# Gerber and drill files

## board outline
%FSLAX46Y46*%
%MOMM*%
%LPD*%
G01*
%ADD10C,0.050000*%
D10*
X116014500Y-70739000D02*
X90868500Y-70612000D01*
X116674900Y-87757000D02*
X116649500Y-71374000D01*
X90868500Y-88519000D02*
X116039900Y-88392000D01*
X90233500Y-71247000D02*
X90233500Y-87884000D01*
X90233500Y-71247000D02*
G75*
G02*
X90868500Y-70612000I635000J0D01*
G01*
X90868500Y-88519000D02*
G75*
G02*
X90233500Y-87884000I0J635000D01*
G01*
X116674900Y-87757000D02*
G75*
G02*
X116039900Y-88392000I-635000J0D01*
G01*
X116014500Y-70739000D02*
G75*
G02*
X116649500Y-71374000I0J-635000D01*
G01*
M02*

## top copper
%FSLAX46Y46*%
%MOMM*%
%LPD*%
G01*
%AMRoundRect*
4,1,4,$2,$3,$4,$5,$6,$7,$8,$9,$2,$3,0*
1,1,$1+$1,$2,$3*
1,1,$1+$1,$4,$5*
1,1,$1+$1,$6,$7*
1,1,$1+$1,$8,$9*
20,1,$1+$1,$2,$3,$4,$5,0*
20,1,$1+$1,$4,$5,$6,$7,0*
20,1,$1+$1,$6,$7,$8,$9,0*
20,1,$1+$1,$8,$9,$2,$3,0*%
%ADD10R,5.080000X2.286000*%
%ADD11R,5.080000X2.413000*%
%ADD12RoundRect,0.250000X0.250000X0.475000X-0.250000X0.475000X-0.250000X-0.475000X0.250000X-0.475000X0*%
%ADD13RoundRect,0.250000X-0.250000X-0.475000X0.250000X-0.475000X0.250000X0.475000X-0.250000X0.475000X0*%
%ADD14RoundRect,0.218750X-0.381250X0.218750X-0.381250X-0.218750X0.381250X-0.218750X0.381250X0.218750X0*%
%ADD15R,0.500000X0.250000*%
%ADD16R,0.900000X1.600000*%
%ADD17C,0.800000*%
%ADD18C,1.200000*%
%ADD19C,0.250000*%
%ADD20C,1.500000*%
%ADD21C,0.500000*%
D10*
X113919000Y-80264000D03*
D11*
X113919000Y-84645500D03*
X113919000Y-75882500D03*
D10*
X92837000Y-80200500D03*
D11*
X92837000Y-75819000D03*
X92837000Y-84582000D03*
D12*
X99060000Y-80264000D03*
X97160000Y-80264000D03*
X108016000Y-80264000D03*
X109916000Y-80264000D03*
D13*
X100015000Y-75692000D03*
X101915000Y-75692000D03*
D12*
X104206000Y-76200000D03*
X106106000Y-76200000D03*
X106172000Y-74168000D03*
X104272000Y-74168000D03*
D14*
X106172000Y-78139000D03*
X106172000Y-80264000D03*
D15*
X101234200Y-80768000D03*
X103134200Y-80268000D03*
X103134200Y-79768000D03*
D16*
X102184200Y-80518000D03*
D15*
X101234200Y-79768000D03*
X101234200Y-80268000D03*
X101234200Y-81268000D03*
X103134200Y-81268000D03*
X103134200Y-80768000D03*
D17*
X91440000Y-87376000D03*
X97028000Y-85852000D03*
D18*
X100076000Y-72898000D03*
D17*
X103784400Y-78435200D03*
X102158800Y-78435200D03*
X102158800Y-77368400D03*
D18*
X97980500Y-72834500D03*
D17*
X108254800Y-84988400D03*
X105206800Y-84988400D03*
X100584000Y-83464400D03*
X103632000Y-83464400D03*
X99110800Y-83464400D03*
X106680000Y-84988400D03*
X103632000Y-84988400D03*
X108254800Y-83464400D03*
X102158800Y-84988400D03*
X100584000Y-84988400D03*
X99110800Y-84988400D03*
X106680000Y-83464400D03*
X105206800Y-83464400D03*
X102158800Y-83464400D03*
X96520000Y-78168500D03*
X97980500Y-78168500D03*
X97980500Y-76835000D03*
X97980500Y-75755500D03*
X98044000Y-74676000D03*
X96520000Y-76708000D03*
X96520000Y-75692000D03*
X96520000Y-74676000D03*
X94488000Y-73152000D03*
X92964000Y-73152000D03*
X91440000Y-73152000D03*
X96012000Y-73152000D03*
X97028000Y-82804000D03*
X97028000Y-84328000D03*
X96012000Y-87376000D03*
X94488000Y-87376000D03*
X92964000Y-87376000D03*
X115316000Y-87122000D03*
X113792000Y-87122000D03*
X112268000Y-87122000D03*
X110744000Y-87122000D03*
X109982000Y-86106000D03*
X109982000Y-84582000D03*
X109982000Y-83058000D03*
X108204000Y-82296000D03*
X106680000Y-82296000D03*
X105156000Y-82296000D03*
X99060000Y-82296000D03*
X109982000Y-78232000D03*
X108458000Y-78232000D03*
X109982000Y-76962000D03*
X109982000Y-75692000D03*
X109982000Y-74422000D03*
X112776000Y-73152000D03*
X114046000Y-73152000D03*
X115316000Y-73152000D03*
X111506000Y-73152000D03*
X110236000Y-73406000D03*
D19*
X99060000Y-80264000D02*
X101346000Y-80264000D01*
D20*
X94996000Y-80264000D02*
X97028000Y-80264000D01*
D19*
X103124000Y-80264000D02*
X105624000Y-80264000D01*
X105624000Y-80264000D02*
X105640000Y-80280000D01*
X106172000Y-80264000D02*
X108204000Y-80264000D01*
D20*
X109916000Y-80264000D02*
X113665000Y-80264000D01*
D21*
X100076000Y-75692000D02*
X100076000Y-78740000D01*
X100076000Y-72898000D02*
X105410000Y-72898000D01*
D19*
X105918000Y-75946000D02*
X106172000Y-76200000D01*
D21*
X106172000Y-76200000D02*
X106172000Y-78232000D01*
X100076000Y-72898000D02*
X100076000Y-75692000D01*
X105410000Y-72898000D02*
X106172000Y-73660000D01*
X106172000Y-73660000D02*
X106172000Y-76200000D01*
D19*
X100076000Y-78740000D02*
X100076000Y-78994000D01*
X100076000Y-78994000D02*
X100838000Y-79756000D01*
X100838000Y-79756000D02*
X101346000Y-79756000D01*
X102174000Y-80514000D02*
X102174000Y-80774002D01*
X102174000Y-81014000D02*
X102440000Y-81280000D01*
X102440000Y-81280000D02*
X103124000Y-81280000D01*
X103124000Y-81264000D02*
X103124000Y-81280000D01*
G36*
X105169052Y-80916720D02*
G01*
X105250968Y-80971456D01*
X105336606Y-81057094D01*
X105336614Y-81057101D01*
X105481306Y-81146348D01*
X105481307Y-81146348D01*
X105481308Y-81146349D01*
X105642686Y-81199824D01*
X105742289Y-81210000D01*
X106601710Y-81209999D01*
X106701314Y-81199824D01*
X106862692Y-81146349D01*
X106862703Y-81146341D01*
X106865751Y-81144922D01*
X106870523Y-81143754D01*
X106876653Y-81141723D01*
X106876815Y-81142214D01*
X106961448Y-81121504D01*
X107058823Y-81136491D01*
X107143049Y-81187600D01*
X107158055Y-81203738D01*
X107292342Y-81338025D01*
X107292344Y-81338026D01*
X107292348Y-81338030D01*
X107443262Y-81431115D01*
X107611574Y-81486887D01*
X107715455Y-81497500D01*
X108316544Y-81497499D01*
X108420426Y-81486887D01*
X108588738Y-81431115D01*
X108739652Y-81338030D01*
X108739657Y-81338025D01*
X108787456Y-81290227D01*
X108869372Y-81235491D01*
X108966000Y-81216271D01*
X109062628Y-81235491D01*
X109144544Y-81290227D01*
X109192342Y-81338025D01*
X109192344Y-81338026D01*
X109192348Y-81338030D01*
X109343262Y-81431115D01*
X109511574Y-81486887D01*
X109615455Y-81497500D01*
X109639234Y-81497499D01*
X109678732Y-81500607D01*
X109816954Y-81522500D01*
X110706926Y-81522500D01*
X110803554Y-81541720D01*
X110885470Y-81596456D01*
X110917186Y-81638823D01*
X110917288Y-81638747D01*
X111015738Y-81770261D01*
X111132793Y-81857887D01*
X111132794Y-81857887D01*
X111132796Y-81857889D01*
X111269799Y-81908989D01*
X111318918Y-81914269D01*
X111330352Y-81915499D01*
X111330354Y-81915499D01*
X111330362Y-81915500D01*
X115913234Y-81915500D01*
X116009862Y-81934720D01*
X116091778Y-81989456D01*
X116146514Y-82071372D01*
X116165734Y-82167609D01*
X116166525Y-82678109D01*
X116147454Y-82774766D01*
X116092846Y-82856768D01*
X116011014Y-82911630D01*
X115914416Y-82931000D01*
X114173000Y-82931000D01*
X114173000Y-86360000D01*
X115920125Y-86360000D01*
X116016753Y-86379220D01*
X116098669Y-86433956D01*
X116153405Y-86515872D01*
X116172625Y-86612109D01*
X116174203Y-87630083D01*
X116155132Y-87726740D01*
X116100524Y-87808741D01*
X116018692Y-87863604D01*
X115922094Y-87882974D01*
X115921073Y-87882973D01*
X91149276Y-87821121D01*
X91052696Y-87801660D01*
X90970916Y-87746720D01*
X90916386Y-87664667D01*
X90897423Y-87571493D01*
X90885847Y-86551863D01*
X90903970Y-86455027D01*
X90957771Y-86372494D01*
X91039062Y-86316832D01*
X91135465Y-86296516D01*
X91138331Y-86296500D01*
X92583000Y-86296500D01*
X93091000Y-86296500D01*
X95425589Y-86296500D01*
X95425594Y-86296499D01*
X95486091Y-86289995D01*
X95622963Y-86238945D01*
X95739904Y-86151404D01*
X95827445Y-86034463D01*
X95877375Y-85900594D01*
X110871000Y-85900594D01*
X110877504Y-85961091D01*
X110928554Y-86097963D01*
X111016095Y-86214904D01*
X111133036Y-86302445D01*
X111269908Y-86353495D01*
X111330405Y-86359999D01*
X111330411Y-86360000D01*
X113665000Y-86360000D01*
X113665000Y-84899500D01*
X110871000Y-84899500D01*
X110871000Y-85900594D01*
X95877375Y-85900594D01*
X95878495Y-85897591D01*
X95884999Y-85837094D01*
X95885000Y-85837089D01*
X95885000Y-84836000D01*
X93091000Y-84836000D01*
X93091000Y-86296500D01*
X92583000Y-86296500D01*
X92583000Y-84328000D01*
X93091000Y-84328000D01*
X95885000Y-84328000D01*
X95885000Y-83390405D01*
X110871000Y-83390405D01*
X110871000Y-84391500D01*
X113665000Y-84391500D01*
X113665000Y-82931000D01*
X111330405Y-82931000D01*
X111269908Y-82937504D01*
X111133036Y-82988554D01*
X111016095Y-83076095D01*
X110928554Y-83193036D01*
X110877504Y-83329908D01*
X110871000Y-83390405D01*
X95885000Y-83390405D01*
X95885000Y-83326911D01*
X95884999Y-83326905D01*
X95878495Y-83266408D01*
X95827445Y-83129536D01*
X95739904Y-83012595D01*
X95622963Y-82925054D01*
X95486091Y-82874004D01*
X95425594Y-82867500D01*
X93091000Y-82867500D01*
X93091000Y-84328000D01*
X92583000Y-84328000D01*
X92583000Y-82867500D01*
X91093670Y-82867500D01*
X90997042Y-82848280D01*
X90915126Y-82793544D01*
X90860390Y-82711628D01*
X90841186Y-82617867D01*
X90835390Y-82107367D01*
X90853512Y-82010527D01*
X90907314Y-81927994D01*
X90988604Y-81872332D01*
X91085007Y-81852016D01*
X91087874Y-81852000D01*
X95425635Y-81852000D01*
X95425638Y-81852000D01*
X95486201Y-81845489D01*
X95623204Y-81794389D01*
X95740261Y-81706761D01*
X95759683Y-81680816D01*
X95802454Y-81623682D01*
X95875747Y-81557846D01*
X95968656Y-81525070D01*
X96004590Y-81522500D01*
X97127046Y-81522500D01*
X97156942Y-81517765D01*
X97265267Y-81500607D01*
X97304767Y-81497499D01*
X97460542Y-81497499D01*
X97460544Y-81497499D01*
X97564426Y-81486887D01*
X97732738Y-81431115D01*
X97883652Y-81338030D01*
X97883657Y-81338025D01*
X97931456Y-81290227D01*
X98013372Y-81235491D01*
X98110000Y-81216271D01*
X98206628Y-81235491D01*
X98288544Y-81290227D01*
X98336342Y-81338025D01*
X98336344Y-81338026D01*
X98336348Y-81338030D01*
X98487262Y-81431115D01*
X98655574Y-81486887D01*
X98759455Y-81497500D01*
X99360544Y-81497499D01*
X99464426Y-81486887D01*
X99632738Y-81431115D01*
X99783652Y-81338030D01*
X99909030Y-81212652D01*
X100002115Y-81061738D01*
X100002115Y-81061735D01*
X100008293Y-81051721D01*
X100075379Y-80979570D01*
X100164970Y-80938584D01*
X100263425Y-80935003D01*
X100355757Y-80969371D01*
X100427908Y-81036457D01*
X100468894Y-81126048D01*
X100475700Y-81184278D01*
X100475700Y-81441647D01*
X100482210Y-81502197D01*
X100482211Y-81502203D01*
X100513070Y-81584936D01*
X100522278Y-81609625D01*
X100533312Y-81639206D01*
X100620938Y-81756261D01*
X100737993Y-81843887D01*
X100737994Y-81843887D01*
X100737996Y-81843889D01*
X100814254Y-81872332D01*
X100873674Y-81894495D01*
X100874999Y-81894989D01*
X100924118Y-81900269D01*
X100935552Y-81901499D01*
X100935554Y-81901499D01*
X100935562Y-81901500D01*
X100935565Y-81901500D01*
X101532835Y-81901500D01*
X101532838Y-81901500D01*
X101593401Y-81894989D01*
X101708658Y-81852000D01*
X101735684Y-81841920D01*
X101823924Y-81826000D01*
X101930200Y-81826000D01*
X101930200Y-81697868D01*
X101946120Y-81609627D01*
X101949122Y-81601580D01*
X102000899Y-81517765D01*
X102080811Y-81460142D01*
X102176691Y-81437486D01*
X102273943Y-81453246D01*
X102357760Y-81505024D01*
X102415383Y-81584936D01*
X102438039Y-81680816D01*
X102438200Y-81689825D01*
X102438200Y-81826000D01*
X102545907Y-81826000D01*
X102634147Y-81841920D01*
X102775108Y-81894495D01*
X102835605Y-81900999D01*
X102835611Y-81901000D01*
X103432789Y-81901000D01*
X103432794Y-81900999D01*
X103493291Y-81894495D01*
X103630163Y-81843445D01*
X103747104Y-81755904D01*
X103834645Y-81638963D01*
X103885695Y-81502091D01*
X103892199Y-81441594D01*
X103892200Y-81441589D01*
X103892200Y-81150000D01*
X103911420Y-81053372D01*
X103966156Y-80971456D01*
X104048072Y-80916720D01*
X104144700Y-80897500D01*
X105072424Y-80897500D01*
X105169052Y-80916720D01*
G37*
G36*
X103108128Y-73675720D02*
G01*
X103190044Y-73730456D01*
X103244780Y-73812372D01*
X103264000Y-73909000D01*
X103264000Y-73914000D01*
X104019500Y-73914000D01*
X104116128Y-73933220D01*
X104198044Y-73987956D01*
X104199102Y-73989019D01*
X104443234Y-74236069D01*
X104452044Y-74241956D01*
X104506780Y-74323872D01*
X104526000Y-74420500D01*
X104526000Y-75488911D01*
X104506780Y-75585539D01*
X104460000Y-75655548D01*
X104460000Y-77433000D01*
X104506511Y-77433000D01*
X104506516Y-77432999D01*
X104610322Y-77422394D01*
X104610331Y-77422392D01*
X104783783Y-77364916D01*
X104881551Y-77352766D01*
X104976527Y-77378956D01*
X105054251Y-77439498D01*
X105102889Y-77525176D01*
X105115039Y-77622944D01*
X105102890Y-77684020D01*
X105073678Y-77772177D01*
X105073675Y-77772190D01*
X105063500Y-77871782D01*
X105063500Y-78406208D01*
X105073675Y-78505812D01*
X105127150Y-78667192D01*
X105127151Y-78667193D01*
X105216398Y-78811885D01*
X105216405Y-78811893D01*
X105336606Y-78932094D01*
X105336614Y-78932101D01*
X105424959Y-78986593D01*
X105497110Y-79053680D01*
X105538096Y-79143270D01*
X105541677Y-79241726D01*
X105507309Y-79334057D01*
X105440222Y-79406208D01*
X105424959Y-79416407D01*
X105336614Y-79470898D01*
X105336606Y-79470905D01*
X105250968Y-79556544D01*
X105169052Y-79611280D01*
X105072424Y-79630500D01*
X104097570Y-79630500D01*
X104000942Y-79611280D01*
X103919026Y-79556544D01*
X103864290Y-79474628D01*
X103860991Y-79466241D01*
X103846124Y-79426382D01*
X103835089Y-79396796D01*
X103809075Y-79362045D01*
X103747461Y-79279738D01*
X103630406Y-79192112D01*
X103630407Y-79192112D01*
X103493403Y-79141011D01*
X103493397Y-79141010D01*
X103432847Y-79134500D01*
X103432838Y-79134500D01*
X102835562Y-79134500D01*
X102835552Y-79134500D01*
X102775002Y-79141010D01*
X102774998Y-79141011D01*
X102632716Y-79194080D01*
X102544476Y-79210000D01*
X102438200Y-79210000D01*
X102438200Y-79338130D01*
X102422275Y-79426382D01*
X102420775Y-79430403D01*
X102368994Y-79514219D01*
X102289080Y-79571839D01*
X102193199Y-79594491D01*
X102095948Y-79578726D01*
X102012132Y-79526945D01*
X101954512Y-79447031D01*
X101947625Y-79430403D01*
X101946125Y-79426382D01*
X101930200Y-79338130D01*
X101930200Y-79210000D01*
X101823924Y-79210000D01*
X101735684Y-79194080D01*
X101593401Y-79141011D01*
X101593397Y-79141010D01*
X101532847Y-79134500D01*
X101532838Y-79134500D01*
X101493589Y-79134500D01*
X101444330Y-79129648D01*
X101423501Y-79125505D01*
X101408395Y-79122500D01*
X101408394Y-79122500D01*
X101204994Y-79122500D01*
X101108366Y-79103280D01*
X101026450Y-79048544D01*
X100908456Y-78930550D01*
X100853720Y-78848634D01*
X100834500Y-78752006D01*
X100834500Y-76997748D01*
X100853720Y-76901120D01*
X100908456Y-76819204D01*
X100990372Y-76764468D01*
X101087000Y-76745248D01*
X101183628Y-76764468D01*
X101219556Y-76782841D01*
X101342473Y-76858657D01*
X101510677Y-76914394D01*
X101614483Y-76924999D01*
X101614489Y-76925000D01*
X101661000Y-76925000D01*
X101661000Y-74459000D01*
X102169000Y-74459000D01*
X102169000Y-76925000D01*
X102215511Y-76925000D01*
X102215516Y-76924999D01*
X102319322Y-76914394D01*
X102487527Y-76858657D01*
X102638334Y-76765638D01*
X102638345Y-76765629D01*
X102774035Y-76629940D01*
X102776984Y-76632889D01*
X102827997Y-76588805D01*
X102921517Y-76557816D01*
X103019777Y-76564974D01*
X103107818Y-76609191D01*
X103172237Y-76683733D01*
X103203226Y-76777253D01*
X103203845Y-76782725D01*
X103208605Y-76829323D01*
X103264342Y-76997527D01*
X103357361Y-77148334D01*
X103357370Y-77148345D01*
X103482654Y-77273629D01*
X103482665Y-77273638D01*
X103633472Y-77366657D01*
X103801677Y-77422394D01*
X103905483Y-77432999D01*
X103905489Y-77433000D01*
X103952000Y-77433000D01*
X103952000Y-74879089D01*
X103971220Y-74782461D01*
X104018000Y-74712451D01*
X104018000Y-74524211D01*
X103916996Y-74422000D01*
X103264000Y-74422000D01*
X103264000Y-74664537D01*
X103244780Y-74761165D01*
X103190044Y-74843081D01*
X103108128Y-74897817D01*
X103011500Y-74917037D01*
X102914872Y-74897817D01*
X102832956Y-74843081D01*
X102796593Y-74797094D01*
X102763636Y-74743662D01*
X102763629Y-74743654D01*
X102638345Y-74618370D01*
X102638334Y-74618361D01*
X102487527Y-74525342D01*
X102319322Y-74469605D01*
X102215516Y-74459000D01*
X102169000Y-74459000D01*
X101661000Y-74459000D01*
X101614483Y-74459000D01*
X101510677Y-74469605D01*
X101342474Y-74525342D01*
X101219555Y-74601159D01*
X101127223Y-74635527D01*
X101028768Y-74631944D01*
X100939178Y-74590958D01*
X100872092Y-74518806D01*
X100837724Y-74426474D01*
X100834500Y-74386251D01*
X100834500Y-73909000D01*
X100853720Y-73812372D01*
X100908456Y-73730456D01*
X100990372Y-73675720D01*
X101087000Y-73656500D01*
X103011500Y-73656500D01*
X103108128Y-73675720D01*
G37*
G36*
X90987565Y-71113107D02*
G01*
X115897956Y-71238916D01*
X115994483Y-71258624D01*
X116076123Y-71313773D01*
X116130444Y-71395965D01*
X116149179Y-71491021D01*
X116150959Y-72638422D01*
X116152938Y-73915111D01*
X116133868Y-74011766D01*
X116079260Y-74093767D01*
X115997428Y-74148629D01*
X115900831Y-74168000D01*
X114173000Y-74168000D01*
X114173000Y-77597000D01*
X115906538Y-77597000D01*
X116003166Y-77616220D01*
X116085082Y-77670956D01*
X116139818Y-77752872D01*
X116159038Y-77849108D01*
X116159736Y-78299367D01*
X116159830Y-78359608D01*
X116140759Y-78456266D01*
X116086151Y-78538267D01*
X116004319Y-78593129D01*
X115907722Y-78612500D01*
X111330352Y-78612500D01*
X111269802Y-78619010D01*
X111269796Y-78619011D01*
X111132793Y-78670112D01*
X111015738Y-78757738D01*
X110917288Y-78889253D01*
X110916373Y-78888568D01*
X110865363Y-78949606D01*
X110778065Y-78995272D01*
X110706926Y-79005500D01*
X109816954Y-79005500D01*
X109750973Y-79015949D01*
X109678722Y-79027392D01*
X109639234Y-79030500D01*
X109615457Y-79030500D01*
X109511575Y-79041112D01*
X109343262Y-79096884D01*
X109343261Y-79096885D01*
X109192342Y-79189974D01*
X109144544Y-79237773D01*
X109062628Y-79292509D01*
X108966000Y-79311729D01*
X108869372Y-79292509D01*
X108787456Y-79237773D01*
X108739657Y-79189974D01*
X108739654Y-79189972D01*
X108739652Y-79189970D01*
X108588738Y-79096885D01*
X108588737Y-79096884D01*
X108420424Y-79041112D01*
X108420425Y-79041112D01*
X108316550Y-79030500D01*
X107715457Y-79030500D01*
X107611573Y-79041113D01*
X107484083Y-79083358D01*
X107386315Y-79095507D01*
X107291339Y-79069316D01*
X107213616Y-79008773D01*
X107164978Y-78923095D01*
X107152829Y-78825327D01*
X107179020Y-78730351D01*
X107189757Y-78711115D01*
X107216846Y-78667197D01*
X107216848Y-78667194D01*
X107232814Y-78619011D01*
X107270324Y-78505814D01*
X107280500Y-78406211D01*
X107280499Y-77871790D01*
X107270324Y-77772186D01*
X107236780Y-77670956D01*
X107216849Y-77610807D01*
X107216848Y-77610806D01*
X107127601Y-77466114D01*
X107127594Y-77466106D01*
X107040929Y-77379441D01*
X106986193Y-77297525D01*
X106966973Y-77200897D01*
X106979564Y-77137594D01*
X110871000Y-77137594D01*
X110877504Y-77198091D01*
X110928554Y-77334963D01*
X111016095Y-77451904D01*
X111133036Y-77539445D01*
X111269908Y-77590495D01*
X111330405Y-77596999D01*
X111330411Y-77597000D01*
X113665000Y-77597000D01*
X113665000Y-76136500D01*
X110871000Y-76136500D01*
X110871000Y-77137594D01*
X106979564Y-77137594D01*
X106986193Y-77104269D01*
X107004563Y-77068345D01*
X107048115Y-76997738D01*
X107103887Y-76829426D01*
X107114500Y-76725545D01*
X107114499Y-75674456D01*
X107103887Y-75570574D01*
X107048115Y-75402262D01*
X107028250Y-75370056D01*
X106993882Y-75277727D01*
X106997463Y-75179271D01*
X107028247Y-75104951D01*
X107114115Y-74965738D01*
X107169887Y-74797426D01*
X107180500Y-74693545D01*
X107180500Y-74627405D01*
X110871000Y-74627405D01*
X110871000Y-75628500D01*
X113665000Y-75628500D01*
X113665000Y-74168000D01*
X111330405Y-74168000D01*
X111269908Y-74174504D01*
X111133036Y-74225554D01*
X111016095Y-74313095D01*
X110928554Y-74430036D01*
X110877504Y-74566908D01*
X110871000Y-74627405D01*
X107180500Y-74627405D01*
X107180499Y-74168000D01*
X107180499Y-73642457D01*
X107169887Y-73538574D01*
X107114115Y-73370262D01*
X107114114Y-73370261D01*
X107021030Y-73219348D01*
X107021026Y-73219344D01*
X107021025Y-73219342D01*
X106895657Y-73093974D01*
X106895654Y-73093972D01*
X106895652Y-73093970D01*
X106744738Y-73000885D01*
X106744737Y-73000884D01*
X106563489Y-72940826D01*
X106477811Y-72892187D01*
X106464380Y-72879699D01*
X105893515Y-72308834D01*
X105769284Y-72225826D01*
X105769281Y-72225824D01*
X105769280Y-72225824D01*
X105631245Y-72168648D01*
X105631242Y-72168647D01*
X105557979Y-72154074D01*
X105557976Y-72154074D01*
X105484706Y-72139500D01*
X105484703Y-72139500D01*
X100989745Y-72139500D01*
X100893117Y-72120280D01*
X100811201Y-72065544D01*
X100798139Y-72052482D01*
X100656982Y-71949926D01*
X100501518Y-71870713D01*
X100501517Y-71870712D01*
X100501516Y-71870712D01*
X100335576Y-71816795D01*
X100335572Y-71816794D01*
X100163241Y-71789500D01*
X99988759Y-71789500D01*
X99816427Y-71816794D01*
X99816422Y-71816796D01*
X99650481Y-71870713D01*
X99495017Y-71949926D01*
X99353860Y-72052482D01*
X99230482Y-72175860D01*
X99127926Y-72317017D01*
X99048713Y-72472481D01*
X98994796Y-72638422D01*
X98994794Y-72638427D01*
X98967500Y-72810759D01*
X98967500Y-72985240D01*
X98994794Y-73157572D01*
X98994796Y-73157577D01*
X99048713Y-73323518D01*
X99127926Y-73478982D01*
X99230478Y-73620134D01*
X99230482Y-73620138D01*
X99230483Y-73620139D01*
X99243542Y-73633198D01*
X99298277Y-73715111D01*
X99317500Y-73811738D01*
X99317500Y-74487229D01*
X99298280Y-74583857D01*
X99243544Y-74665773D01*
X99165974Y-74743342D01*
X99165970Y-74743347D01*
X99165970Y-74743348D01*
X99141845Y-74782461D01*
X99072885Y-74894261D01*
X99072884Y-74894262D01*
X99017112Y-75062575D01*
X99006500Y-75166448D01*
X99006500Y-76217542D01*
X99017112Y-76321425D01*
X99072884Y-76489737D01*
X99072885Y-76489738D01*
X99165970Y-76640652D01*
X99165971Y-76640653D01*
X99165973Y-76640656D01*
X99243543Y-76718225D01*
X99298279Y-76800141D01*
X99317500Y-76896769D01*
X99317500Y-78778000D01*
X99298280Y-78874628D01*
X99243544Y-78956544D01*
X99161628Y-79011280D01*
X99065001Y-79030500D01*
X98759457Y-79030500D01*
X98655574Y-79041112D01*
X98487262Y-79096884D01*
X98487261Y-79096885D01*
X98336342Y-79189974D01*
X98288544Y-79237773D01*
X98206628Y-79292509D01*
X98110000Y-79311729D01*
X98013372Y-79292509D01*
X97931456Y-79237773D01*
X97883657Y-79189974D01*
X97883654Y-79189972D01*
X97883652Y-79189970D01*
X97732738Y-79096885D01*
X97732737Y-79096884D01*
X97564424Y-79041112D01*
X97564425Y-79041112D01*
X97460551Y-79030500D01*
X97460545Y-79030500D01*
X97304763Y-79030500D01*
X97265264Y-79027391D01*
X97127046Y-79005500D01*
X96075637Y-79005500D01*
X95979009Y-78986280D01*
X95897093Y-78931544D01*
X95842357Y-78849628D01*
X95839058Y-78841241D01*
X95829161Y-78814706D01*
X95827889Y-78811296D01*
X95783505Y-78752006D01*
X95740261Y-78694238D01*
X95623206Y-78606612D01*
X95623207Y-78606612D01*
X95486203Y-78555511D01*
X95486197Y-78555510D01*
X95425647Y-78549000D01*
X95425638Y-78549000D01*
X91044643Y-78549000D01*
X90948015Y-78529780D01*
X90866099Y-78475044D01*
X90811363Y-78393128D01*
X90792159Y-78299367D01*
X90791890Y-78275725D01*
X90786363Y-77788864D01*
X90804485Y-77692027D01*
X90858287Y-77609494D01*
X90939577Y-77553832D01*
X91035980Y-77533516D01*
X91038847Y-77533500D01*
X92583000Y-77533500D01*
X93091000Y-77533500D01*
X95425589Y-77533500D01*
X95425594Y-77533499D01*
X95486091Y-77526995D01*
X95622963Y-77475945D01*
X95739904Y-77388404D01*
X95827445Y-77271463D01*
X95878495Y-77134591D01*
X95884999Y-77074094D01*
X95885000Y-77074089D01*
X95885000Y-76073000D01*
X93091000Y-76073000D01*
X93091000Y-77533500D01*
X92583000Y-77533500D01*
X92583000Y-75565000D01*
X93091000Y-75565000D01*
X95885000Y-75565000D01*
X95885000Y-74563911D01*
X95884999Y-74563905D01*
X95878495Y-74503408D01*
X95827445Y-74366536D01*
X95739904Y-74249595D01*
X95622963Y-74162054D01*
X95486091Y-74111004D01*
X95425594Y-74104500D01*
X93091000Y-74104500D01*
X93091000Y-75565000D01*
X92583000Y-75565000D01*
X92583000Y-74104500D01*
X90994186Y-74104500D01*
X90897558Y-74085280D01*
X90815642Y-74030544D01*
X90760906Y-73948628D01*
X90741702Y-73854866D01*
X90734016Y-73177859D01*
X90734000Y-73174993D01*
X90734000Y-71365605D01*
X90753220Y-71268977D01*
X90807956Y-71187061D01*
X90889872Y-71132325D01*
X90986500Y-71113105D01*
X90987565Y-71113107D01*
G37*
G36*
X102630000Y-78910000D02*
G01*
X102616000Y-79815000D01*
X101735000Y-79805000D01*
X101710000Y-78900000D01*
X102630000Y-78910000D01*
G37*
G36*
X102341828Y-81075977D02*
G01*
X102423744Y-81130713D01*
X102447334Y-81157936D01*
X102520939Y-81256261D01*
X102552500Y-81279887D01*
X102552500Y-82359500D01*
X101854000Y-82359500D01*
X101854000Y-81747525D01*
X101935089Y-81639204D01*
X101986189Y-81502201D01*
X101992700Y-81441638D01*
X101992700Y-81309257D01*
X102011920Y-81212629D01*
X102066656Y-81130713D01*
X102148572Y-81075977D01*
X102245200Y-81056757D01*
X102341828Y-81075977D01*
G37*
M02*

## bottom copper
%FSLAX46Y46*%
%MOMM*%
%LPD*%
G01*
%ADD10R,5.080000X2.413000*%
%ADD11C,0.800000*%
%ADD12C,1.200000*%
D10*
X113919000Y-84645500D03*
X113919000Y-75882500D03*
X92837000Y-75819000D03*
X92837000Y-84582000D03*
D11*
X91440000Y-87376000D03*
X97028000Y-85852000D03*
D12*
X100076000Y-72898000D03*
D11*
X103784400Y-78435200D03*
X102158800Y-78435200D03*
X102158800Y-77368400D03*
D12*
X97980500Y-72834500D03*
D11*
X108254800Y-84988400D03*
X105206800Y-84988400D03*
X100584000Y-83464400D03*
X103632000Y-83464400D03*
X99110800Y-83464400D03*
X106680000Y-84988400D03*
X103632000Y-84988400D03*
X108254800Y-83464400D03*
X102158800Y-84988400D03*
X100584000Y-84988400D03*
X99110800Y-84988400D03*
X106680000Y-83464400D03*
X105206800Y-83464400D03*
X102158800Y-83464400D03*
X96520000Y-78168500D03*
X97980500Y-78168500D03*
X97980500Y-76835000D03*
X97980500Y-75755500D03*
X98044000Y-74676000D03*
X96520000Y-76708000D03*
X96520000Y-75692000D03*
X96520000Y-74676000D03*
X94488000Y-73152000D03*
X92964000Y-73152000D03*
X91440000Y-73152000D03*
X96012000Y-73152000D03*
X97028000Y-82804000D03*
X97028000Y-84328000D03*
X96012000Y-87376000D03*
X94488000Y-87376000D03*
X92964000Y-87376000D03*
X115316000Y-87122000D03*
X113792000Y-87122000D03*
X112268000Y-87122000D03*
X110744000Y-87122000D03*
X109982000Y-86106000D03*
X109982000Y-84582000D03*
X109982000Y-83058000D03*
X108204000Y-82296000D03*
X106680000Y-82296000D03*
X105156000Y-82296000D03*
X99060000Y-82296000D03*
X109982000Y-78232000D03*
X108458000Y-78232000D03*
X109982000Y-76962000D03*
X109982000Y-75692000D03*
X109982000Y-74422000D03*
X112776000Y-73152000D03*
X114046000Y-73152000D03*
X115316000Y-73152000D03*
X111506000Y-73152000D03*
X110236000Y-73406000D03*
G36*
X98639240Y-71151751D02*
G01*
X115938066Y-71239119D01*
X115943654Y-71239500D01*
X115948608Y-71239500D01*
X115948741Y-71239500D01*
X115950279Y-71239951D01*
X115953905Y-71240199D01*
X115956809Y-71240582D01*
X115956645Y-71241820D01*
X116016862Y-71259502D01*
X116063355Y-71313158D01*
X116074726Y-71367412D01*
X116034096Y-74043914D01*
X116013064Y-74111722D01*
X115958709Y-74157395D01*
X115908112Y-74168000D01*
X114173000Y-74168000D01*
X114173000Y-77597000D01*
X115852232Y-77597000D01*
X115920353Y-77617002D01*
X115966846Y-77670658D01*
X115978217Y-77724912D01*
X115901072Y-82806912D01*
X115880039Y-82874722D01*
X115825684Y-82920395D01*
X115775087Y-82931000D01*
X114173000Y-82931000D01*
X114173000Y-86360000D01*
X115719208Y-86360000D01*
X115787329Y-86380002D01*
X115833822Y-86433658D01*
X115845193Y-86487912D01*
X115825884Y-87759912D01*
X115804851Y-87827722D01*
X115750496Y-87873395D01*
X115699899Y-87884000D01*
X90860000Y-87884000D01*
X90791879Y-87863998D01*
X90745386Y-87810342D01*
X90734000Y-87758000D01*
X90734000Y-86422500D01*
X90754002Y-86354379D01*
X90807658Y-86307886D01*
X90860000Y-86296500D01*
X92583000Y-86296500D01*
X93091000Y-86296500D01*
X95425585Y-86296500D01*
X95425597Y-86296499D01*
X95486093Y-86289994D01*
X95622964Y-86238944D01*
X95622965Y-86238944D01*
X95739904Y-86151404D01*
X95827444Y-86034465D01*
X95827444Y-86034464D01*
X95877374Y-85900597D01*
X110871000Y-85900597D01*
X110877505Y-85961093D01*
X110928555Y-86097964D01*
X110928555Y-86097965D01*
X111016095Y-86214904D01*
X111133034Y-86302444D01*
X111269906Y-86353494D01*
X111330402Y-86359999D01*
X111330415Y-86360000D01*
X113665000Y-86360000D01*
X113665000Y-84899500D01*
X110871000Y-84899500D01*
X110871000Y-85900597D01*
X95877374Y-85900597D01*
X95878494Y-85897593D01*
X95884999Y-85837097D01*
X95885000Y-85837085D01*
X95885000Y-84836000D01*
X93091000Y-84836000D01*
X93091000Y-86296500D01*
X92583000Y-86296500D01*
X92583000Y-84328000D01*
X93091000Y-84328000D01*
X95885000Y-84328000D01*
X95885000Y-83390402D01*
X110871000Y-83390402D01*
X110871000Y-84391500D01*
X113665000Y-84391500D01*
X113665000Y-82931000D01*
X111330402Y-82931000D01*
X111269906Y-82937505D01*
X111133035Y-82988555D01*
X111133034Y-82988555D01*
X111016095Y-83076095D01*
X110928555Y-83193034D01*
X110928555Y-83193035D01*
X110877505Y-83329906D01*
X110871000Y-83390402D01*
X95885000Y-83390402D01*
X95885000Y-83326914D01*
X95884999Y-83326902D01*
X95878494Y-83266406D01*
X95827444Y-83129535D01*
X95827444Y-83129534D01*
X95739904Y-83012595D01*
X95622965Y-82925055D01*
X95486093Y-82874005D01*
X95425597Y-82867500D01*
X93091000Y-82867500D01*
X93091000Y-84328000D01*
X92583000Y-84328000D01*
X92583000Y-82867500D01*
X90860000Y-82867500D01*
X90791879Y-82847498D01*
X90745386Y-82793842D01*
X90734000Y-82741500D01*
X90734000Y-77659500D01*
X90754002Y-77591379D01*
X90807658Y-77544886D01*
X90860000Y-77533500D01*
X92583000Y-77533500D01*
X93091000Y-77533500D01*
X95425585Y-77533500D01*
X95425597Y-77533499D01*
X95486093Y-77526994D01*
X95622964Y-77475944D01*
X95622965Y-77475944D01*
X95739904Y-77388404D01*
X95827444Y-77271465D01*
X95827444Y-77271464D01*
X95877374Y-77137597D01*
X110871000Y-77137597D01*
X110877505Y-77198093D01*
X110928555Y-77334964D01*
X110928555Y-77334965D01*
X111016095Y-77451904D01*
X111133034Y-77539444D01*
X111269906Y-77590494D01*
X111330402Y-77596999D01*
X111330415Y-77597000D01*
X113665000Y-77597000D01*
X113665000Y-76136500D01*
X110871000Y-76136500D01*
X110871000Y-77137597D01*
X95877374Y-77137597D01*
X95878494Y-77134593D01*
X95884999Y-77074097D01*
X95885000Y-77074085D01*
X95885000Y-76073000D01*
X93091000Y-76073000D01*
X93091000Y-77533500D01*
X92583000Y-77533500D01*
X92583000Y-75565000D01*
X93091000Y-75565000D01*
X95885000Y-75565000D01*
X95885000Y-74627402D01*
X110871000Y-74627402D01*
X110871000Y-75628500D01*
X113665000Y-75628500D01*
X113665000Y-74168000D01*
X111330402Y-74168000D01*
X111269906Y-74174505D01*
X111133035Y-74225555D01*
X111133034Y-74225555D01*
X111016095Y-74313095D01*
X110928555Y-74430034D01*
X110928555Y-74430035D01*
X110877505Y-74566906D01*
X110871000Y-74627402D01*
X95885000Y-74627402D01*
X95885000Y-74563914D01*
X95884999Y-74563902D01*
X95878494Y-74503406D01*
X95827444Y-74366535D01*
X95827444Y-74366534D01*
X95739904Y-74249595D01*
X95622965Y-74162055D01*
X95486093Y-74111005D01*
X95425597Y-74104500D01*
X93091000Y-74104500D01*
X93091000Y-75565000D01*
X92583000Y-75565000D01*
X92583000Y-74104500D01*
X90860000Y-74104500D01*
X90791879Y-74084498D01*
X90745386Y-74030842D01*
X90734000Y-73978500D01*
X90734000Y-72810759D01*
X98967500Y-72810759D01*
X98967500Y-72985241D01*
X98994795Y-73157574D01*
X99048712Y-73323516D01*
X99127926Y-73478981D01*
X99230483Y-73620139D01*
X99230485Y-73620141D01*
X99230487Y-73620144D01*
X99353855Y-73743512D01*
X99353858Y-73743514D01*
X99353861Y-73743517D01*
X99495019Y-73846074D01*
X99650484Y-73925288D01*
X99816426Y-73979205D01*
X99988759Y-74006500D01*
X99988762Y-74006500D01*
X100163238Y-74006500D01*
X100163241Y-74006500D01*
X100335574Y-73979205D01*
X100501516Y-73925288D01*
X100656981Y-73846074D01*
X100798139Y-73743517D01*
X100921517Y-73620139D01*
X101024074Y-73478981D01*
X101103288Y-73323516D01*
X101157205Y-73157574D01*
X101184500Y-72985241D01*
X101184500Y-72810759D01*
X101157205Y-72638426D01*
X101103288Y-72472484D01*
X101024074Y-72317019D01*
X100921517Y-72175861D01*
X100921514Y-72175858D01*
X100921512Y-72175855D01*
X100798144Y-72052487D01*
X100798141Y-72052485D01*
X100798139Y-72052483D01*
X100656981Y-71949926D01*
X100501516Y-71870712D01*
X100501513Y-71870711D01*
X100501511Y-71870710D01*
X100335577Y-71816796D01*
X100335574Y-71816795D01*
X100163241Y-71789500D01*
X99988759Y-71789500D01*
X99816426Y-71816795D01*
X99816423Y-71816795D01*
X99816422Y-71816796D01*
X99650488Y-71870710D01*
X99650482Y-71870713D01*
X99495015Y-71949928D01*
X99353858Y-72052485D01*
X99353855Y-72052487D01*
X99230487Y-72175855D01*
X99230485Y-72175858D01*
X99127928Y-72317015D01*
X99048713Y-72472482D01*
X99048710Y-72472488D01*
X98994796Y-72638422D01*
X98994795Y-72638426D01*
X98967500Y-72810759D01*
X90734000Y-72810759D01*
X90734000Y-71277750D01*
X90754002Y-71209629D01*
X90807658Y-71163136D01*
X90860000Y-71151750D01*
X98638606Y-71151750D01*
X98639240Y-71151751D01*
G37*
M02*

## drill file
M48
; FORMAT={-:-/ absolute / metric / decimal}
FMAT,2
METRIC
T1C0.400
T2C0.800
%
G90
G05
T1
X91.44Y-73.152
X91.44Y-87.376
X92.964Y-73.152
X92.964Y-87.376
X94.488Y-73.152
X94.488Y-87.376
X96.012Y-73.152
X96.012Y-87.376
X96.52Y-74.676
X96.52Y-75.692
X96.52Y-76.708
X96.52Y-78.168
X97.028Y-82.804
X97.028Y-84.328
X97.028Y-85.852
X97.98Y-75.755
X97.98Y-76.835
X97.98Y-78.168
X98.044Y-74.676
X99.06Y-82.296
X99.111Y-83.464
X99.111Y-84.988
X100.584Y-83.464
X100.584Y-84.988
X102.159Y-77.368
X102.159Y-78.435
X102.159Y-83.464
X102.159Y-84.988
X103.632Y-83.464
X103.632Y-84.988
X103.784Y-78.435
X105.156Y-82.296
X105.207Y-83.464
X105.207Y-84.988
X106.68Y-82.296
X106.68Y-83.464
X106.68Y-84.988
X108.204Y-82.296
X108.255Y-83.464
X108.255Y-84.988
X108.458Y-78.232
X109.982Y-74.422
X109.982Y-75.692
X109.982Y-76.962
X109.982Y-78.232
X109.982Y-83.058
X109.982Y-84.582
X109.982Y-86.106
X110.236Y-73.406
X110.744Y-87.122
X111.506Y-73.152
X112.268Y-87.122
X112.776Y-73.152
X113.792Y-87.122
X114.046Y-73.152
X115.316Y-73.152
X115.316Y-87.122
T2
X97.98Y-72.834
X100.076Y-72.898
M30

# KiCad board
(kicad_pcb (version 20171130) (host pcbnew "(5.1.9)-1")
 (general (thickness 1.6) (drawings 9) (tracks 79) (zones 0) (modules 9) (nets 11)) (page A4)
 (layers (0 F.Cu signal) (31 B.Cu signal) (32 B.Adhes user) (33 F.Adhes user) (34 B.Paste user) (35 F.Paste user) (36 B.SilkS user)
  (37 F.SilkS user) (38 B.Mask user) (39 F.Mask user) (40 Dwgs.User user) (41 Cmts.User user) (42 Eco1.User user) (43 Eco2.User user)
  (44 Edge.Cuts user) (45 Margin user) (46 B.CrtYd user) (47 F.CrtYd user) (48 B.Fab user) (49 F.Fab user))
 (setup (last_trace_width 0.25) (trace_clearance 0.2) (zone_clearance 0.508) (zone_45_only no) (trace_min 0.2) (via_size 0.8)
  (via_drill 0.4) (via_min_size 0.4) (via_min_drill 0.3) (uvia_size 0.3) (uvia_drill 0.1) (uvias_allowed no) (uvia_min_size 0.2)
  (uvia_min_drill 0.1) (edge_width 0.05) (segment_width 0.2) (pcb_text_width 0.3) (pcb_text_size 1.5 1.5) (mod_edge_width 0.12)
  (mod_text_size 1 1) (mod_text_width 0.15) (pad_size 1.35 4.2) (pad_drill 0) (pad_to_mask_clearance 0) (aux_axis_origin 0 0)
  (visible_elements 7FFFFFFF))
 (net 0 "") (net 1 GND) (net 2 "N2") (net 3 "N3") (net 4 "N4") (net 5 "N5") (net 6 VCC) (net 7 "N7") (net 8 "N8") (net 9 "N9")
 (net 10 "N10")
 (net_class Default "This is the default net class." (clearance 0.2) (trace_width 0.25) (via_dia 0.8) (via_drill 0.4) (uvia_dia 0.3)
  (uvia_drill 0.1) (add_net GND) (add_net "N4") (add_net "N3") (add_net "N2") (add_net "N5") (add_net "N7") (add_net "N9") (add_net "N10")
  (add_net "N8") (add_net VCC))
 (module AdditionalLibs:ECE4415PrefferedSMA (layer F.Cu) (at 113.919 80.264 270)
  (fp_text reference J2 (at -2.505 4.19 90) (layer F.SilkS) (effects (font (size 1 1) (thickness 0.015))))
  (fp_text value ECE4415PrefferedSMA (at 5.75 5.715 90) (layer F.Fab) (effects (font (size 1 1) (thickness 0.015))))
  (pad S4 smd rect (at 4.3815 0 270) (size 2.413 5.08) (layers B.Cu B.Paste B.Mask) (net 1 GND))
  (pad S3 smd rect (at -4.3815 0 270) (size 2.413 5.08) (layers B.Cu B.Paste B.Mask) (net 1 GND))
  (pad 1 smd rect (at 0 0 270) (size 2.286 5.08) (layers F.Cu F.Paste F.Mask) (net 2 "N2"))
  (pad S2 smd rect (at 4.3815 0 270) (size 2.413 5.08) (layers F.Cu F.Paste F.Mask) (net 1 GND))
  (pad S1 smd rect (at -4.3815 0 270) (size 2.413 5.08) (layers F.Cu F.Paste F.Mask) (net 1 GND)))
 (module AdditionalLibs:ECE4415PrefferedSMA (layer F.Cu) (at 92.837 80.2005 90)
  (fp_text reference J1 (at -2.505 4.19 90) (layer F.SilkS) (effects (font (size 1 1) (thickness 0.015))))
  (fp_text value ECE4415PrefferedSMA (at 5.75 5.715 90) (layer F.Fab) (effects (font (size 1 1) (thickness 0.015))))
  (pad S4 smd rect (at 4.3815 0 90) (size 2.413 5.08) (layers B.Cu B.Paste B.Mask) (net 1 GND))
  (pad S3 smd rect (at -4.3815 0 90) (size 2.413 5.08) (layers B.Cu B.Paste B.Mask) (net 1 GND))
  (pad 1 smd rect (at 0 0 90) (size 2.286 5.08) (layers F.Cu F.Paste F.Mask) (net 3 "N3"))
  (pad S2 smd rect (at 4.3815 0 90) (size 2.413 5.08) (layers F.Cu F.Paste F.Mask) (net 1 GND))
  (pad S1 smd rect (at -4.3815 0 90) (size 2.413 5.08) (layers F.Cu F.Paste F.Mask) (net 1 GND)))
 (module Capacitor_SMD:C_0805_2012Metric (layer F.Cu) (at 98.11 80.264 180)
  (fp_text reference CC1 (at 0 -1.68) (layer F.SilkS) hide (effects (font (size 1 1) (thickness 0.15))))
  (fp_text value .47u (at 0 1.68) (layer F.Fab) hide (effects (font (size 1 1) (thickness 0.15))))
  (pad 1 smd roundrect (at -0.95 0 180) (size 1 1.45) (layers F.Cu F.Paste F.Mask) (roundrect_rratio 0.25) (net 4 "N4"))
  (pad 2 smd roundrect (at 0.95 0 180) (size 1 1.45) (layers F.Cu F.Paste F.Mask) (roundrect_rratio 0.25) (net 3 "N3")))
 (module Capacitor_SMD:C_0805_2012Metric (layer F.Cu) (at 108.966 80.264 180)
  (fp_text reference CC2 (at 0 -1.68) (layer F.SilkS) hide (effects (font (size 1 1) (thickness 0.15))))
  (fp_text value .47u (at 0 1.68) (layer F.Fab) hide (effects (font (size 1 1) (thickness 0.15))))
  (pad 2 smd roundrect (at 0.95 0 180) (size 1 1.45) (layers F.Cu F.Paste F.Mask) (roundrect_rratio 0.25) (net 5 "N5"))
  (pad 1 smd roundrect (at -0.95 0 180) (size 1 1.45) (layers F.Cu F.Paste F.Mask) (roundrect_rratio 0.25) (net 2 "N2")))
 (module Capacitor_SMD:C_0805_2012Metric (layer F.Cu) (at 100.965 75.692)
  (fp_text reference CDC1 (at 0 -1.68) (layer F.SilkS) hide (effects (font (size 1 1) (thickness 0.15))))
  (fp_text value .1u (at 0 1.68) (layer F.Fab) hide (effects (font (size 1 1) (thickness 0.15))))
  (pad 1 smd roundrect (at -0.95 0) (size 1 1.45) (layers F.Cu F.Paste F.Mask) (roundrect_rratio 0.25) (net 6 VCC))
  (pad 2 smd roundrect (at 0.95 0) (size 1 1.45) (layers F.Cu F.Paste F.Mask) (roundrect_rratio 0.25) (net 1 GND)))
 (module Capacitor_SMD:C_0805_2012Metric (layer F.Cu) (at 105.156 76.2 180)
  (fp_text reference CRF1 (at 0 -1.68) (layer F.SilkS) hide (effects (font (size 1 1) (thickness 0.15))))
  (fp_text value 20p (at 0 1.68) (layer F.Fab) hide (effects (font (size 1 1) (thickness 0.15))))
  (pad 2 smd roundrect (at 0.95 0 180) (size 1 1.45) (layers F.Cu F.Paste F.Mask) (roundrect_rratio 0.25) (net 1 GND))
  (pad 1 smd roundrect (at -0.95 0 180) (size 1 1.45) (layers F.Cu F.Paste F.Mask) (roundrect_rratio 0.25) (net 6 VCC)))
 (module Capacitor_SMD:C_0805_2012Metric (layer F.Cu) (at 105.222 74.168 180)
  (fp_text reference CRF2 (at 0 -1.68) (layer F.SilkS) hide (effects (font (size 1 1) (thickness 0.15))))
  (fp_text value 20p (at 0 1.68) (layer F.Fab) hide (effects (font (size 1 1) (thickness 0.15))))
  (pad 1 smd roundrect (at -0.95 0 180) (size 1 1.45) (layers F.Cu F.Paste F.Mask) (roundrect_rratio 0.25) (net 6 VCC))
  (pad 2 smd roundrect (at 0.95 0 180) (size 1 1.45) (layers F.Cu F.Paste F.Mask) (roundrect_rratio 0.25) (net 1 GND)))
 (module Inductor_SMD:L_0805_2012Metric (layer F.Cu) (at 106.172 79.2015 270)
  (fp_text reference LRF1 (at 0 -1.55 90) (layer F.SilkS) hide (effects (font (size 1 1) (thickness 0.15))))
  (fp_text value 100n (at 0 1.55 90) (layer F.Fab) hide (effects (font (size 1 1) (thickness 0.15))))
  (pad 1 smd roundrect (at -1.0625 0 270) (size 0.875 1.2) (layers F.Cu F.Paste F.Mask) (roundrect_rratio 0.25) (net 6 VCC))
  (pad 2 smd roundrect (at 1.0625 0 270) (size 0.875 1.2) (layers F.Cu F.Paste F.Mask) (roundrect_rratio 0.25) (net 5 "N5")))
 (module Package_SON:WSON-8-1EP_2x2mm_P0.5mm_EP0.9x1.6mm (layer F.Cu) (at 102.1842 80.518)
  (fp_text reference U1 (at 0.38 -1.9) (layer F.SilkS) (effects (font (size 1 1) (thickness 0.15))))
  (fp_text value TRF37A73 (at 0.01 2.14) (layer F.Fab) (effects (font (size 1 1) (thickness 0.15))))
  (pad 3 smd rect (at -0.95 0.25) (size 0.5 0.25) (layers F.Cu F.Paste F.Mask) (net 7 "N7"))
  (pad 7 smd rect (at 0.95 -0.25) (size 0.5 0.25) (layers F.Cu F.Paste F.Mask) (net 5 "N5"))
  (pad 8 smd rect (at 0.95 -0.75) (size 0.5 0.25) (layers F.Cu F.Paste F.Mask) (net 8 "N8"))
  (pad 9 smd rect (at 0 0) (size 0.9 1.6) (layers F.Cu F.Mask) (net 1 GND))
  (pad 1 smd rect (at -0.95 -0.75) (size 0.5 0.25) (layers F.Cu F.Paste F.Mask) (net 6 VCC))
  (pad 2 smd rect (at -0.95 -0.25) (size 0.5 0.25) (layers F.Cu F.Paste F.Mask) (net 4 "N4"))
  (pad 4 smd rect (at -0.95 0.75) (size 0.5 0.25) (layers F.Cu F.Paste F.Mask) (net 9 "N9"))
  (pad 5 smd rect (at 0.95 0.75) (size 0.5 0.25) (layers F.Cu F.Paste F.Mask) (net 1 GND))
  (pad 6 smd rect (at 0.95 0.25) (size 0.5 0.25) (layers F.Cu F.Paste F.Mask) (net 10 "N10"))
  (pad "" smd rect (at 0 0.4) (size 0.75 0.65) (layers F.Paste))
  (pad "" smd rect (at 0 -0.4) (size 0.75 0.65) (layers F.Paste)))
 (gr_line (start 116.0145 70.739) (end 90.8685 70.612) (layer Edge.Cuts) (width 0.05))
 (gr_line (start 116.6749 87.757) (end 116.6495 71.374) (layer Edge.Cuts) (width 0.05))
 (gr_line (start 90.8685 88.519) (end 116.0399 88.392) (layer Edge.Cuts) (width 0.05))
 (gr_line (start 90.2335 71.247) (end 90.2335 87.884) (layer Edge.Cuts) (width 0.05))
 (gr_arc (start 90.8685 71.247) (end 90.8685 70.612) (angle -90) (layer Edge.Cuts) (width 0.05))
 (gr_arc (start 90.8685 87.884) (end 90.2335 87.884) (angle -90) (layer Edge.Cuts) (width 0.05))
 (gr_arc (start 116.0399 87.757) (end 116.0399 88.392) (angle -90) (layer Edge.Cuts) (width 0.05))
 (gr_arc (start 116.0145 71.374) (end 116.6495 71.374) (angle -90) (layer Edge.Cuts) (width 0.05))
 (via (at 91.44 87.376) (size 0.8) (drill 0.4) (layers F.Cu B.Cu) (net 1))
 (via (at 97.028 85.852) (size 0.8) (drill 0.4) (layers F.Cu B.Cu) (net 1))
 (segment (start 99.06 80.264) (end 101.346 80.264) (width 0.25) (layer F.Cu) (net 4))
 (segment (start 94.996 80.264) (end 97.028 80.264) (width 1.5) (layer F.Cu) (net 3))
 (segment (start 103.124 80.264) (end 105.624 80.264) (width 0.25) (layer F.Cu) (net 5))
 (segment (start 105.624 80.264) (end 105.64 80.28) (width 0.25) (layer F.Cu) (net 5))
 (segment (start 106.172 80.264) (end 108.204 80.264) (width 0.25) (layer F.Cu) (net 5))
 (segment (start 109.916 80.264) (end 113.665 80.264) (width 1.5) (layer F.Cu) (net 2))
 (via (at 100.076 72.898) (size 1.2) (drill 0.8) (layers F.Cu B.Cu) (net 6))
 (segment (start 100.076 75.692) (end 100.076 78.74) (width 0.5) (layer F.Cu) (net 6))
 (segment (start 100.076 72.898) (end 105.41 72.898) (width 0.5) (layer F.Cu) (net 6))
 (segment (start 105.918 75.946) (end 106.172 76.2) (width 0.25) (layer F.Cu) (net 6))
 (segment (start 106.172 76.2) (end 106.172 78.232) (width 0.5) (layer F.Cu) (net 6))
 (segment (start 100.076 72.898) (end 100.076 75.692) (width 0.5) (layer F.Cu) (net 6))
 (segment (start 105.41 72.898) (end 106.172 73.66) (width 0.5) (layer F.Cu) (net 6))
 (segment (start 106.172 73.66) (end 106.172 76.2) (width 0.5) (layer F.Cu) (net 6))
 (segment (start 100.076 78.74) (end 100.076 78.994) (width 0.25) (layer F.Cu) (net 6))
 (segment (start 100.076 78.994) (end 100.838 79.756) (width 0.25) (layer F.Cu) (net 6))
 (segment (start 100.838 79.756) (end 101.346 79.756) (width 0.25) (layer F.Cu) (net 6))
 (via (at 103.7844 78.4352) (size 0.8) (drill 0.4) (layers F.Cu B.Cu) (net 1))
 (via (at 102.1588 78.4352) (size 0.8) (drill 0.4) (layers F.Cu B.Cu) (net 1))
 (via (at 102.1588 77.3684) (size 0.8) (drill 0.4) (layers F.Cu B.Cu) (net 1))
 (segment (start 102.174 80.514) (end 102.174 80.774002) (width 0.25) (layer F.Cu) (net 1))
 (segment (start 102.174 81.014) (end 102.44 81.28) (width 0.25) (layer F.Cu) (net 1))
 (segment (start 102.44 81.28) (end 103.124 81.28) (width 0.25) (layer F.Cu) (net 1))
 (via (at 97.9805 72.8345) (size 1.2) (drill 0.8) (layers F.Cu B.Cu) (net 1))
 (via (at 108.2548 84.9884) (size 0.8) (drill 0.4) (layers F.Cu B.Cu) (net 1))
 (via (at 105.2068 84.9884) (size 0.8) (drill 0.4) (layers F.Cu B.Cu) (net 1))
 (via (at 100.584 83.4644) (size 0.8) (drill 0.4) (layers F.Cu B.Cu) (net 1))
 (via (at 103.632 83.4644) (size 0.8) (drill 0.4) (layers F.Cu B.Cu) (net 1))
 (via (at 99.1108 83.4644) (size 0.8) (drill 0.4) (layers F.Cu B.Cu) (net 1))
 (via (at 106.68 84.9884) (size 0.8) (drill 0.4) (layers F.Cu B.Cu) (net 1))
 (via (at 103.632 84.9884) (size 0.8) (drill 0.4) (layers F.Cu B.Cu) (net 1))
 (via (at 108.2548 83.4644) (size 0.8) (drill 0.4) (layers F.Cu B.Cu) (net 1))
 (via (at 102.1588 84.9884) (size 0.8) (drill 0.4) (layers F.Cu B.Cu) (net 1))
 (via (at 100.584 84.9884) (size 0.8) (drill 0.4) (layers F.Cu B.Cu) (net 1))
 (via (at 99.1108 84.9884) (size 0.8) (drill 0.4) (layers F.Cu B.Cu) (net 1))
 (via (at 106.68 83.4644) (size 0.8) (drill 0.4) (layers F.Cu B.Cu) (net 1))
 (via (at 105.2068 83.4644) (size 0.8) (drill 0.4) (layers F.Cu B.Cu) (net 1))
 (via (at 102.1588 83.4644) (size 0.8) (drill 0.4) (layers F.Cu B.Cu) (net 1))
 (segment (start 103.124 81.264) (end 103.124 81.28) (width 0.25) (layer F.Cu) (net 1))
 (via (at 96.52 78.1685) (size 0.8) (drill 0.4) (layers F.Cu B.Cu) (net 1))
 (via (at 97.9805 78.1685) (size 0.8) (drill 0.4) (layers F.Cu B.Cu) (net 1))
 (via (at 97.9805 76.835) (size 0.8) (drill 0.4) (layers F.Cu B.Cu) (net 1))
 (via (at 97.9805 75.7555) (size 0.8) (drill 0.4) (layers F.Cu B.Cu) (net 1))
 (via (at 98.044 74.676) (size 0.8) (drill 0.4) (layers F.Cu B.Cu) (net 1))
 (via (at 96.52 76.708) (size 0.8) (drill 0.4) (layers F.Cu B.Cu) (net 1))
 (via (at 96.52 75.692) (size 0.8) (drill 0.4) (layers F.Cu B.Cu) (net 1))
 (via (at 96.52 74.676) (size 0.8) (drill 0.4) (layers F.Cu B.Cu) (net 1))
 (via (at 94.488 73.152) (size 0.8) (drill 0.4) (layers F.Cu B.Cu) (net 1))
 (via (at 92.964 73.152) (size 0.8) (drill 0.4) (layers F.Cu B.Cu) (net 1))
 (via (at 91.44 73.152) (size 0.8) (drill 0.4) (layers F.Cu B.Cu) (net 1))
 (via (at 96.012 73.152) (size 0.8) (drill 0.4) (layers F.Cu B.Cu) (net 1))
 (via (at 97.028 82.804) (size 0.8) (drill 0.4) (layers F.Cu B.Cu) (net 1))
 (via (at 97.028 84.328) (size 0.8) (drill 0.4) (layers F.Cu B.Cu) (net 1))
 (via (at 96.012 87.376) (size 0.8) (drill 0.4) (layers F.Cu B.Cu) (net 1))
 (via (at 94.488 87.376) (size 0.8) (drill 0.4) (layers F.Cu B.Cu) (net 1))
 (via (at 92.964 87.376) (size 0.8) (drill 0.4) (layers F.Cu B.Cu) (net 1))
 (via (at 115.316 87.122) (size 0.8) (drill 0.4) (layers F.Cu B.Cu) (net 1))
 (via (at 113.792 87.122) (size 0.8) (drill 0.4) (layers F.Cu B.Cu) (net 1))
 (via (at 112.268 87.122) (size 0.8) (drill 0.4) (layers F.Cu B.Cu) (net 1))
 (via (at 110.744 87.122) (size 0.8) (drill 0.4) (layers F.Cu B.Cu) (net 1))
 (via (at 109.982 86.106) (size 0.8) (drill 0.4) (layers F.Cu B.Cu) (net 1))
 (via (at 109.982 84.582) (size 0.8) (drill 0.4) (layers F.Cu B.Cu) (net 1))
 (via (at 109.982 83.058) (size 0.8) (drill 0.4) (layers F.Cu B.Cu) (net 1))
 (via (at 108.204 82.296) (size 0.8) (drill 0.4) (layers F.Cu B.Cu) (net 1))
 (via (at 106.68 82.296) (size 0.8) (drill 0.4) (layers F.Cu B.Cu) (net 1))
 (via (at 105.156 82.296) (size 0.8) (drill 0.4) (layers F.Cu B.Cu) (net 1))
 (via (at 99.06 82.296) (size 0.8) (drill 0.4) (layers F.Cu B.Cu) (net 1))
 (via (at 109.982 78.232) (size 0.8) (drill 0.4) (layers F.Cu B.Cu) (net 1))
 (via (at 108.458 78.232) (size 0.8) (drill 0.4) (layers F.Cu B.Cu) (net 1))
 (via (at 109.982 76.962) (size 0.8) (drill 0.4) (layers F.Cu B.Cu) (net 1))
 (via (at 109.982 75.692) (size 0.8) (drill 0.4) (layers F.Cu B.Cu) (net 1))
 (via (at 109.982 74.422) (size 0.8) (drill 0.4) (layers F.Cu B.Cu) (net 1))
 (via (at 112.776 73.152) (size 0.8) (drill 0.4) (layers F.Cu B.Cu) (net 1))
 (via (at 114.046 73.152) (size 0.8) (drill 0.4) (layers F.Cu B.Cu) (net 1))
 (via (at 115.316 73.152) (size 0.8) (drill 0.4) (layers F.Cu B.Cu) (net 1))
 (via (at 111.506 73.152) (size 0.8) (drill 0.4) (layers F.Cu B.Cu) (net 1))
 (via (at 110.236 73.406) (size 0.8) (drill 0.4) (layers F.Cu B.Cu) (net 1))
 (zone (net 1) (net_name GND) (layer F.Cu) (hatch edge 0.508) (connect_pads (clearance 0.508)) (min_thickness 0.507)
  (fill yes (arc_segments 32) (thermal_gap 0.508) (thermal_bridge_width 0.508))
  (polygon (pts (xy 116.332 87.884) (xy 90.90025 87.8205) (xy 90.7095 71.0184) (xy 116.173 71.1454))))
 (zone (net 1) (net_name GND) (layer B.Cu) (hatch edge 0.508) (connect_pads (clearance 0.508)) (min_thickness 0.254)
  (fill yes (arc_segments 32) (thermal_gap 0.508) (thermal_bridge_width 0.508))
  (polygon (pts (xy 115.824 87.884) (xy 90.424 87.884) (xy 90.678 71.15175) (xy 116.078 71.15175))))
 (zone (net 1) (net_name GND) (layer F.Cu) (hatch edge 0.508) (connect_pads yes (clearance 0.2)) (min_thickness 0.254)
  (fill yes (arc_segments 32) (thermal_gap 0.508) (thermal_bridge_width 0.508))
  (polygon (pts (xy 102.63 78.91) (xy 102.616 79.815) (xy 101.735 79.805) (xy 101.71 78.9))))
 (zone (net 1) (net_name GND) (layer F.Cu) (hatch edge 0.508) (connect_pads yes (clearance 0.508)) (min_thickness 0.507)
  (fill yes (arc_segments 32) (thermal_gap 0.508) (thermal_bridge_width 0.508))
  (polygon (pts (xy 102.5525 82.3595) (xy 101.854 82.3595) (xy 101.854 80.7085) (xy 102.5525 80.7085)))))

